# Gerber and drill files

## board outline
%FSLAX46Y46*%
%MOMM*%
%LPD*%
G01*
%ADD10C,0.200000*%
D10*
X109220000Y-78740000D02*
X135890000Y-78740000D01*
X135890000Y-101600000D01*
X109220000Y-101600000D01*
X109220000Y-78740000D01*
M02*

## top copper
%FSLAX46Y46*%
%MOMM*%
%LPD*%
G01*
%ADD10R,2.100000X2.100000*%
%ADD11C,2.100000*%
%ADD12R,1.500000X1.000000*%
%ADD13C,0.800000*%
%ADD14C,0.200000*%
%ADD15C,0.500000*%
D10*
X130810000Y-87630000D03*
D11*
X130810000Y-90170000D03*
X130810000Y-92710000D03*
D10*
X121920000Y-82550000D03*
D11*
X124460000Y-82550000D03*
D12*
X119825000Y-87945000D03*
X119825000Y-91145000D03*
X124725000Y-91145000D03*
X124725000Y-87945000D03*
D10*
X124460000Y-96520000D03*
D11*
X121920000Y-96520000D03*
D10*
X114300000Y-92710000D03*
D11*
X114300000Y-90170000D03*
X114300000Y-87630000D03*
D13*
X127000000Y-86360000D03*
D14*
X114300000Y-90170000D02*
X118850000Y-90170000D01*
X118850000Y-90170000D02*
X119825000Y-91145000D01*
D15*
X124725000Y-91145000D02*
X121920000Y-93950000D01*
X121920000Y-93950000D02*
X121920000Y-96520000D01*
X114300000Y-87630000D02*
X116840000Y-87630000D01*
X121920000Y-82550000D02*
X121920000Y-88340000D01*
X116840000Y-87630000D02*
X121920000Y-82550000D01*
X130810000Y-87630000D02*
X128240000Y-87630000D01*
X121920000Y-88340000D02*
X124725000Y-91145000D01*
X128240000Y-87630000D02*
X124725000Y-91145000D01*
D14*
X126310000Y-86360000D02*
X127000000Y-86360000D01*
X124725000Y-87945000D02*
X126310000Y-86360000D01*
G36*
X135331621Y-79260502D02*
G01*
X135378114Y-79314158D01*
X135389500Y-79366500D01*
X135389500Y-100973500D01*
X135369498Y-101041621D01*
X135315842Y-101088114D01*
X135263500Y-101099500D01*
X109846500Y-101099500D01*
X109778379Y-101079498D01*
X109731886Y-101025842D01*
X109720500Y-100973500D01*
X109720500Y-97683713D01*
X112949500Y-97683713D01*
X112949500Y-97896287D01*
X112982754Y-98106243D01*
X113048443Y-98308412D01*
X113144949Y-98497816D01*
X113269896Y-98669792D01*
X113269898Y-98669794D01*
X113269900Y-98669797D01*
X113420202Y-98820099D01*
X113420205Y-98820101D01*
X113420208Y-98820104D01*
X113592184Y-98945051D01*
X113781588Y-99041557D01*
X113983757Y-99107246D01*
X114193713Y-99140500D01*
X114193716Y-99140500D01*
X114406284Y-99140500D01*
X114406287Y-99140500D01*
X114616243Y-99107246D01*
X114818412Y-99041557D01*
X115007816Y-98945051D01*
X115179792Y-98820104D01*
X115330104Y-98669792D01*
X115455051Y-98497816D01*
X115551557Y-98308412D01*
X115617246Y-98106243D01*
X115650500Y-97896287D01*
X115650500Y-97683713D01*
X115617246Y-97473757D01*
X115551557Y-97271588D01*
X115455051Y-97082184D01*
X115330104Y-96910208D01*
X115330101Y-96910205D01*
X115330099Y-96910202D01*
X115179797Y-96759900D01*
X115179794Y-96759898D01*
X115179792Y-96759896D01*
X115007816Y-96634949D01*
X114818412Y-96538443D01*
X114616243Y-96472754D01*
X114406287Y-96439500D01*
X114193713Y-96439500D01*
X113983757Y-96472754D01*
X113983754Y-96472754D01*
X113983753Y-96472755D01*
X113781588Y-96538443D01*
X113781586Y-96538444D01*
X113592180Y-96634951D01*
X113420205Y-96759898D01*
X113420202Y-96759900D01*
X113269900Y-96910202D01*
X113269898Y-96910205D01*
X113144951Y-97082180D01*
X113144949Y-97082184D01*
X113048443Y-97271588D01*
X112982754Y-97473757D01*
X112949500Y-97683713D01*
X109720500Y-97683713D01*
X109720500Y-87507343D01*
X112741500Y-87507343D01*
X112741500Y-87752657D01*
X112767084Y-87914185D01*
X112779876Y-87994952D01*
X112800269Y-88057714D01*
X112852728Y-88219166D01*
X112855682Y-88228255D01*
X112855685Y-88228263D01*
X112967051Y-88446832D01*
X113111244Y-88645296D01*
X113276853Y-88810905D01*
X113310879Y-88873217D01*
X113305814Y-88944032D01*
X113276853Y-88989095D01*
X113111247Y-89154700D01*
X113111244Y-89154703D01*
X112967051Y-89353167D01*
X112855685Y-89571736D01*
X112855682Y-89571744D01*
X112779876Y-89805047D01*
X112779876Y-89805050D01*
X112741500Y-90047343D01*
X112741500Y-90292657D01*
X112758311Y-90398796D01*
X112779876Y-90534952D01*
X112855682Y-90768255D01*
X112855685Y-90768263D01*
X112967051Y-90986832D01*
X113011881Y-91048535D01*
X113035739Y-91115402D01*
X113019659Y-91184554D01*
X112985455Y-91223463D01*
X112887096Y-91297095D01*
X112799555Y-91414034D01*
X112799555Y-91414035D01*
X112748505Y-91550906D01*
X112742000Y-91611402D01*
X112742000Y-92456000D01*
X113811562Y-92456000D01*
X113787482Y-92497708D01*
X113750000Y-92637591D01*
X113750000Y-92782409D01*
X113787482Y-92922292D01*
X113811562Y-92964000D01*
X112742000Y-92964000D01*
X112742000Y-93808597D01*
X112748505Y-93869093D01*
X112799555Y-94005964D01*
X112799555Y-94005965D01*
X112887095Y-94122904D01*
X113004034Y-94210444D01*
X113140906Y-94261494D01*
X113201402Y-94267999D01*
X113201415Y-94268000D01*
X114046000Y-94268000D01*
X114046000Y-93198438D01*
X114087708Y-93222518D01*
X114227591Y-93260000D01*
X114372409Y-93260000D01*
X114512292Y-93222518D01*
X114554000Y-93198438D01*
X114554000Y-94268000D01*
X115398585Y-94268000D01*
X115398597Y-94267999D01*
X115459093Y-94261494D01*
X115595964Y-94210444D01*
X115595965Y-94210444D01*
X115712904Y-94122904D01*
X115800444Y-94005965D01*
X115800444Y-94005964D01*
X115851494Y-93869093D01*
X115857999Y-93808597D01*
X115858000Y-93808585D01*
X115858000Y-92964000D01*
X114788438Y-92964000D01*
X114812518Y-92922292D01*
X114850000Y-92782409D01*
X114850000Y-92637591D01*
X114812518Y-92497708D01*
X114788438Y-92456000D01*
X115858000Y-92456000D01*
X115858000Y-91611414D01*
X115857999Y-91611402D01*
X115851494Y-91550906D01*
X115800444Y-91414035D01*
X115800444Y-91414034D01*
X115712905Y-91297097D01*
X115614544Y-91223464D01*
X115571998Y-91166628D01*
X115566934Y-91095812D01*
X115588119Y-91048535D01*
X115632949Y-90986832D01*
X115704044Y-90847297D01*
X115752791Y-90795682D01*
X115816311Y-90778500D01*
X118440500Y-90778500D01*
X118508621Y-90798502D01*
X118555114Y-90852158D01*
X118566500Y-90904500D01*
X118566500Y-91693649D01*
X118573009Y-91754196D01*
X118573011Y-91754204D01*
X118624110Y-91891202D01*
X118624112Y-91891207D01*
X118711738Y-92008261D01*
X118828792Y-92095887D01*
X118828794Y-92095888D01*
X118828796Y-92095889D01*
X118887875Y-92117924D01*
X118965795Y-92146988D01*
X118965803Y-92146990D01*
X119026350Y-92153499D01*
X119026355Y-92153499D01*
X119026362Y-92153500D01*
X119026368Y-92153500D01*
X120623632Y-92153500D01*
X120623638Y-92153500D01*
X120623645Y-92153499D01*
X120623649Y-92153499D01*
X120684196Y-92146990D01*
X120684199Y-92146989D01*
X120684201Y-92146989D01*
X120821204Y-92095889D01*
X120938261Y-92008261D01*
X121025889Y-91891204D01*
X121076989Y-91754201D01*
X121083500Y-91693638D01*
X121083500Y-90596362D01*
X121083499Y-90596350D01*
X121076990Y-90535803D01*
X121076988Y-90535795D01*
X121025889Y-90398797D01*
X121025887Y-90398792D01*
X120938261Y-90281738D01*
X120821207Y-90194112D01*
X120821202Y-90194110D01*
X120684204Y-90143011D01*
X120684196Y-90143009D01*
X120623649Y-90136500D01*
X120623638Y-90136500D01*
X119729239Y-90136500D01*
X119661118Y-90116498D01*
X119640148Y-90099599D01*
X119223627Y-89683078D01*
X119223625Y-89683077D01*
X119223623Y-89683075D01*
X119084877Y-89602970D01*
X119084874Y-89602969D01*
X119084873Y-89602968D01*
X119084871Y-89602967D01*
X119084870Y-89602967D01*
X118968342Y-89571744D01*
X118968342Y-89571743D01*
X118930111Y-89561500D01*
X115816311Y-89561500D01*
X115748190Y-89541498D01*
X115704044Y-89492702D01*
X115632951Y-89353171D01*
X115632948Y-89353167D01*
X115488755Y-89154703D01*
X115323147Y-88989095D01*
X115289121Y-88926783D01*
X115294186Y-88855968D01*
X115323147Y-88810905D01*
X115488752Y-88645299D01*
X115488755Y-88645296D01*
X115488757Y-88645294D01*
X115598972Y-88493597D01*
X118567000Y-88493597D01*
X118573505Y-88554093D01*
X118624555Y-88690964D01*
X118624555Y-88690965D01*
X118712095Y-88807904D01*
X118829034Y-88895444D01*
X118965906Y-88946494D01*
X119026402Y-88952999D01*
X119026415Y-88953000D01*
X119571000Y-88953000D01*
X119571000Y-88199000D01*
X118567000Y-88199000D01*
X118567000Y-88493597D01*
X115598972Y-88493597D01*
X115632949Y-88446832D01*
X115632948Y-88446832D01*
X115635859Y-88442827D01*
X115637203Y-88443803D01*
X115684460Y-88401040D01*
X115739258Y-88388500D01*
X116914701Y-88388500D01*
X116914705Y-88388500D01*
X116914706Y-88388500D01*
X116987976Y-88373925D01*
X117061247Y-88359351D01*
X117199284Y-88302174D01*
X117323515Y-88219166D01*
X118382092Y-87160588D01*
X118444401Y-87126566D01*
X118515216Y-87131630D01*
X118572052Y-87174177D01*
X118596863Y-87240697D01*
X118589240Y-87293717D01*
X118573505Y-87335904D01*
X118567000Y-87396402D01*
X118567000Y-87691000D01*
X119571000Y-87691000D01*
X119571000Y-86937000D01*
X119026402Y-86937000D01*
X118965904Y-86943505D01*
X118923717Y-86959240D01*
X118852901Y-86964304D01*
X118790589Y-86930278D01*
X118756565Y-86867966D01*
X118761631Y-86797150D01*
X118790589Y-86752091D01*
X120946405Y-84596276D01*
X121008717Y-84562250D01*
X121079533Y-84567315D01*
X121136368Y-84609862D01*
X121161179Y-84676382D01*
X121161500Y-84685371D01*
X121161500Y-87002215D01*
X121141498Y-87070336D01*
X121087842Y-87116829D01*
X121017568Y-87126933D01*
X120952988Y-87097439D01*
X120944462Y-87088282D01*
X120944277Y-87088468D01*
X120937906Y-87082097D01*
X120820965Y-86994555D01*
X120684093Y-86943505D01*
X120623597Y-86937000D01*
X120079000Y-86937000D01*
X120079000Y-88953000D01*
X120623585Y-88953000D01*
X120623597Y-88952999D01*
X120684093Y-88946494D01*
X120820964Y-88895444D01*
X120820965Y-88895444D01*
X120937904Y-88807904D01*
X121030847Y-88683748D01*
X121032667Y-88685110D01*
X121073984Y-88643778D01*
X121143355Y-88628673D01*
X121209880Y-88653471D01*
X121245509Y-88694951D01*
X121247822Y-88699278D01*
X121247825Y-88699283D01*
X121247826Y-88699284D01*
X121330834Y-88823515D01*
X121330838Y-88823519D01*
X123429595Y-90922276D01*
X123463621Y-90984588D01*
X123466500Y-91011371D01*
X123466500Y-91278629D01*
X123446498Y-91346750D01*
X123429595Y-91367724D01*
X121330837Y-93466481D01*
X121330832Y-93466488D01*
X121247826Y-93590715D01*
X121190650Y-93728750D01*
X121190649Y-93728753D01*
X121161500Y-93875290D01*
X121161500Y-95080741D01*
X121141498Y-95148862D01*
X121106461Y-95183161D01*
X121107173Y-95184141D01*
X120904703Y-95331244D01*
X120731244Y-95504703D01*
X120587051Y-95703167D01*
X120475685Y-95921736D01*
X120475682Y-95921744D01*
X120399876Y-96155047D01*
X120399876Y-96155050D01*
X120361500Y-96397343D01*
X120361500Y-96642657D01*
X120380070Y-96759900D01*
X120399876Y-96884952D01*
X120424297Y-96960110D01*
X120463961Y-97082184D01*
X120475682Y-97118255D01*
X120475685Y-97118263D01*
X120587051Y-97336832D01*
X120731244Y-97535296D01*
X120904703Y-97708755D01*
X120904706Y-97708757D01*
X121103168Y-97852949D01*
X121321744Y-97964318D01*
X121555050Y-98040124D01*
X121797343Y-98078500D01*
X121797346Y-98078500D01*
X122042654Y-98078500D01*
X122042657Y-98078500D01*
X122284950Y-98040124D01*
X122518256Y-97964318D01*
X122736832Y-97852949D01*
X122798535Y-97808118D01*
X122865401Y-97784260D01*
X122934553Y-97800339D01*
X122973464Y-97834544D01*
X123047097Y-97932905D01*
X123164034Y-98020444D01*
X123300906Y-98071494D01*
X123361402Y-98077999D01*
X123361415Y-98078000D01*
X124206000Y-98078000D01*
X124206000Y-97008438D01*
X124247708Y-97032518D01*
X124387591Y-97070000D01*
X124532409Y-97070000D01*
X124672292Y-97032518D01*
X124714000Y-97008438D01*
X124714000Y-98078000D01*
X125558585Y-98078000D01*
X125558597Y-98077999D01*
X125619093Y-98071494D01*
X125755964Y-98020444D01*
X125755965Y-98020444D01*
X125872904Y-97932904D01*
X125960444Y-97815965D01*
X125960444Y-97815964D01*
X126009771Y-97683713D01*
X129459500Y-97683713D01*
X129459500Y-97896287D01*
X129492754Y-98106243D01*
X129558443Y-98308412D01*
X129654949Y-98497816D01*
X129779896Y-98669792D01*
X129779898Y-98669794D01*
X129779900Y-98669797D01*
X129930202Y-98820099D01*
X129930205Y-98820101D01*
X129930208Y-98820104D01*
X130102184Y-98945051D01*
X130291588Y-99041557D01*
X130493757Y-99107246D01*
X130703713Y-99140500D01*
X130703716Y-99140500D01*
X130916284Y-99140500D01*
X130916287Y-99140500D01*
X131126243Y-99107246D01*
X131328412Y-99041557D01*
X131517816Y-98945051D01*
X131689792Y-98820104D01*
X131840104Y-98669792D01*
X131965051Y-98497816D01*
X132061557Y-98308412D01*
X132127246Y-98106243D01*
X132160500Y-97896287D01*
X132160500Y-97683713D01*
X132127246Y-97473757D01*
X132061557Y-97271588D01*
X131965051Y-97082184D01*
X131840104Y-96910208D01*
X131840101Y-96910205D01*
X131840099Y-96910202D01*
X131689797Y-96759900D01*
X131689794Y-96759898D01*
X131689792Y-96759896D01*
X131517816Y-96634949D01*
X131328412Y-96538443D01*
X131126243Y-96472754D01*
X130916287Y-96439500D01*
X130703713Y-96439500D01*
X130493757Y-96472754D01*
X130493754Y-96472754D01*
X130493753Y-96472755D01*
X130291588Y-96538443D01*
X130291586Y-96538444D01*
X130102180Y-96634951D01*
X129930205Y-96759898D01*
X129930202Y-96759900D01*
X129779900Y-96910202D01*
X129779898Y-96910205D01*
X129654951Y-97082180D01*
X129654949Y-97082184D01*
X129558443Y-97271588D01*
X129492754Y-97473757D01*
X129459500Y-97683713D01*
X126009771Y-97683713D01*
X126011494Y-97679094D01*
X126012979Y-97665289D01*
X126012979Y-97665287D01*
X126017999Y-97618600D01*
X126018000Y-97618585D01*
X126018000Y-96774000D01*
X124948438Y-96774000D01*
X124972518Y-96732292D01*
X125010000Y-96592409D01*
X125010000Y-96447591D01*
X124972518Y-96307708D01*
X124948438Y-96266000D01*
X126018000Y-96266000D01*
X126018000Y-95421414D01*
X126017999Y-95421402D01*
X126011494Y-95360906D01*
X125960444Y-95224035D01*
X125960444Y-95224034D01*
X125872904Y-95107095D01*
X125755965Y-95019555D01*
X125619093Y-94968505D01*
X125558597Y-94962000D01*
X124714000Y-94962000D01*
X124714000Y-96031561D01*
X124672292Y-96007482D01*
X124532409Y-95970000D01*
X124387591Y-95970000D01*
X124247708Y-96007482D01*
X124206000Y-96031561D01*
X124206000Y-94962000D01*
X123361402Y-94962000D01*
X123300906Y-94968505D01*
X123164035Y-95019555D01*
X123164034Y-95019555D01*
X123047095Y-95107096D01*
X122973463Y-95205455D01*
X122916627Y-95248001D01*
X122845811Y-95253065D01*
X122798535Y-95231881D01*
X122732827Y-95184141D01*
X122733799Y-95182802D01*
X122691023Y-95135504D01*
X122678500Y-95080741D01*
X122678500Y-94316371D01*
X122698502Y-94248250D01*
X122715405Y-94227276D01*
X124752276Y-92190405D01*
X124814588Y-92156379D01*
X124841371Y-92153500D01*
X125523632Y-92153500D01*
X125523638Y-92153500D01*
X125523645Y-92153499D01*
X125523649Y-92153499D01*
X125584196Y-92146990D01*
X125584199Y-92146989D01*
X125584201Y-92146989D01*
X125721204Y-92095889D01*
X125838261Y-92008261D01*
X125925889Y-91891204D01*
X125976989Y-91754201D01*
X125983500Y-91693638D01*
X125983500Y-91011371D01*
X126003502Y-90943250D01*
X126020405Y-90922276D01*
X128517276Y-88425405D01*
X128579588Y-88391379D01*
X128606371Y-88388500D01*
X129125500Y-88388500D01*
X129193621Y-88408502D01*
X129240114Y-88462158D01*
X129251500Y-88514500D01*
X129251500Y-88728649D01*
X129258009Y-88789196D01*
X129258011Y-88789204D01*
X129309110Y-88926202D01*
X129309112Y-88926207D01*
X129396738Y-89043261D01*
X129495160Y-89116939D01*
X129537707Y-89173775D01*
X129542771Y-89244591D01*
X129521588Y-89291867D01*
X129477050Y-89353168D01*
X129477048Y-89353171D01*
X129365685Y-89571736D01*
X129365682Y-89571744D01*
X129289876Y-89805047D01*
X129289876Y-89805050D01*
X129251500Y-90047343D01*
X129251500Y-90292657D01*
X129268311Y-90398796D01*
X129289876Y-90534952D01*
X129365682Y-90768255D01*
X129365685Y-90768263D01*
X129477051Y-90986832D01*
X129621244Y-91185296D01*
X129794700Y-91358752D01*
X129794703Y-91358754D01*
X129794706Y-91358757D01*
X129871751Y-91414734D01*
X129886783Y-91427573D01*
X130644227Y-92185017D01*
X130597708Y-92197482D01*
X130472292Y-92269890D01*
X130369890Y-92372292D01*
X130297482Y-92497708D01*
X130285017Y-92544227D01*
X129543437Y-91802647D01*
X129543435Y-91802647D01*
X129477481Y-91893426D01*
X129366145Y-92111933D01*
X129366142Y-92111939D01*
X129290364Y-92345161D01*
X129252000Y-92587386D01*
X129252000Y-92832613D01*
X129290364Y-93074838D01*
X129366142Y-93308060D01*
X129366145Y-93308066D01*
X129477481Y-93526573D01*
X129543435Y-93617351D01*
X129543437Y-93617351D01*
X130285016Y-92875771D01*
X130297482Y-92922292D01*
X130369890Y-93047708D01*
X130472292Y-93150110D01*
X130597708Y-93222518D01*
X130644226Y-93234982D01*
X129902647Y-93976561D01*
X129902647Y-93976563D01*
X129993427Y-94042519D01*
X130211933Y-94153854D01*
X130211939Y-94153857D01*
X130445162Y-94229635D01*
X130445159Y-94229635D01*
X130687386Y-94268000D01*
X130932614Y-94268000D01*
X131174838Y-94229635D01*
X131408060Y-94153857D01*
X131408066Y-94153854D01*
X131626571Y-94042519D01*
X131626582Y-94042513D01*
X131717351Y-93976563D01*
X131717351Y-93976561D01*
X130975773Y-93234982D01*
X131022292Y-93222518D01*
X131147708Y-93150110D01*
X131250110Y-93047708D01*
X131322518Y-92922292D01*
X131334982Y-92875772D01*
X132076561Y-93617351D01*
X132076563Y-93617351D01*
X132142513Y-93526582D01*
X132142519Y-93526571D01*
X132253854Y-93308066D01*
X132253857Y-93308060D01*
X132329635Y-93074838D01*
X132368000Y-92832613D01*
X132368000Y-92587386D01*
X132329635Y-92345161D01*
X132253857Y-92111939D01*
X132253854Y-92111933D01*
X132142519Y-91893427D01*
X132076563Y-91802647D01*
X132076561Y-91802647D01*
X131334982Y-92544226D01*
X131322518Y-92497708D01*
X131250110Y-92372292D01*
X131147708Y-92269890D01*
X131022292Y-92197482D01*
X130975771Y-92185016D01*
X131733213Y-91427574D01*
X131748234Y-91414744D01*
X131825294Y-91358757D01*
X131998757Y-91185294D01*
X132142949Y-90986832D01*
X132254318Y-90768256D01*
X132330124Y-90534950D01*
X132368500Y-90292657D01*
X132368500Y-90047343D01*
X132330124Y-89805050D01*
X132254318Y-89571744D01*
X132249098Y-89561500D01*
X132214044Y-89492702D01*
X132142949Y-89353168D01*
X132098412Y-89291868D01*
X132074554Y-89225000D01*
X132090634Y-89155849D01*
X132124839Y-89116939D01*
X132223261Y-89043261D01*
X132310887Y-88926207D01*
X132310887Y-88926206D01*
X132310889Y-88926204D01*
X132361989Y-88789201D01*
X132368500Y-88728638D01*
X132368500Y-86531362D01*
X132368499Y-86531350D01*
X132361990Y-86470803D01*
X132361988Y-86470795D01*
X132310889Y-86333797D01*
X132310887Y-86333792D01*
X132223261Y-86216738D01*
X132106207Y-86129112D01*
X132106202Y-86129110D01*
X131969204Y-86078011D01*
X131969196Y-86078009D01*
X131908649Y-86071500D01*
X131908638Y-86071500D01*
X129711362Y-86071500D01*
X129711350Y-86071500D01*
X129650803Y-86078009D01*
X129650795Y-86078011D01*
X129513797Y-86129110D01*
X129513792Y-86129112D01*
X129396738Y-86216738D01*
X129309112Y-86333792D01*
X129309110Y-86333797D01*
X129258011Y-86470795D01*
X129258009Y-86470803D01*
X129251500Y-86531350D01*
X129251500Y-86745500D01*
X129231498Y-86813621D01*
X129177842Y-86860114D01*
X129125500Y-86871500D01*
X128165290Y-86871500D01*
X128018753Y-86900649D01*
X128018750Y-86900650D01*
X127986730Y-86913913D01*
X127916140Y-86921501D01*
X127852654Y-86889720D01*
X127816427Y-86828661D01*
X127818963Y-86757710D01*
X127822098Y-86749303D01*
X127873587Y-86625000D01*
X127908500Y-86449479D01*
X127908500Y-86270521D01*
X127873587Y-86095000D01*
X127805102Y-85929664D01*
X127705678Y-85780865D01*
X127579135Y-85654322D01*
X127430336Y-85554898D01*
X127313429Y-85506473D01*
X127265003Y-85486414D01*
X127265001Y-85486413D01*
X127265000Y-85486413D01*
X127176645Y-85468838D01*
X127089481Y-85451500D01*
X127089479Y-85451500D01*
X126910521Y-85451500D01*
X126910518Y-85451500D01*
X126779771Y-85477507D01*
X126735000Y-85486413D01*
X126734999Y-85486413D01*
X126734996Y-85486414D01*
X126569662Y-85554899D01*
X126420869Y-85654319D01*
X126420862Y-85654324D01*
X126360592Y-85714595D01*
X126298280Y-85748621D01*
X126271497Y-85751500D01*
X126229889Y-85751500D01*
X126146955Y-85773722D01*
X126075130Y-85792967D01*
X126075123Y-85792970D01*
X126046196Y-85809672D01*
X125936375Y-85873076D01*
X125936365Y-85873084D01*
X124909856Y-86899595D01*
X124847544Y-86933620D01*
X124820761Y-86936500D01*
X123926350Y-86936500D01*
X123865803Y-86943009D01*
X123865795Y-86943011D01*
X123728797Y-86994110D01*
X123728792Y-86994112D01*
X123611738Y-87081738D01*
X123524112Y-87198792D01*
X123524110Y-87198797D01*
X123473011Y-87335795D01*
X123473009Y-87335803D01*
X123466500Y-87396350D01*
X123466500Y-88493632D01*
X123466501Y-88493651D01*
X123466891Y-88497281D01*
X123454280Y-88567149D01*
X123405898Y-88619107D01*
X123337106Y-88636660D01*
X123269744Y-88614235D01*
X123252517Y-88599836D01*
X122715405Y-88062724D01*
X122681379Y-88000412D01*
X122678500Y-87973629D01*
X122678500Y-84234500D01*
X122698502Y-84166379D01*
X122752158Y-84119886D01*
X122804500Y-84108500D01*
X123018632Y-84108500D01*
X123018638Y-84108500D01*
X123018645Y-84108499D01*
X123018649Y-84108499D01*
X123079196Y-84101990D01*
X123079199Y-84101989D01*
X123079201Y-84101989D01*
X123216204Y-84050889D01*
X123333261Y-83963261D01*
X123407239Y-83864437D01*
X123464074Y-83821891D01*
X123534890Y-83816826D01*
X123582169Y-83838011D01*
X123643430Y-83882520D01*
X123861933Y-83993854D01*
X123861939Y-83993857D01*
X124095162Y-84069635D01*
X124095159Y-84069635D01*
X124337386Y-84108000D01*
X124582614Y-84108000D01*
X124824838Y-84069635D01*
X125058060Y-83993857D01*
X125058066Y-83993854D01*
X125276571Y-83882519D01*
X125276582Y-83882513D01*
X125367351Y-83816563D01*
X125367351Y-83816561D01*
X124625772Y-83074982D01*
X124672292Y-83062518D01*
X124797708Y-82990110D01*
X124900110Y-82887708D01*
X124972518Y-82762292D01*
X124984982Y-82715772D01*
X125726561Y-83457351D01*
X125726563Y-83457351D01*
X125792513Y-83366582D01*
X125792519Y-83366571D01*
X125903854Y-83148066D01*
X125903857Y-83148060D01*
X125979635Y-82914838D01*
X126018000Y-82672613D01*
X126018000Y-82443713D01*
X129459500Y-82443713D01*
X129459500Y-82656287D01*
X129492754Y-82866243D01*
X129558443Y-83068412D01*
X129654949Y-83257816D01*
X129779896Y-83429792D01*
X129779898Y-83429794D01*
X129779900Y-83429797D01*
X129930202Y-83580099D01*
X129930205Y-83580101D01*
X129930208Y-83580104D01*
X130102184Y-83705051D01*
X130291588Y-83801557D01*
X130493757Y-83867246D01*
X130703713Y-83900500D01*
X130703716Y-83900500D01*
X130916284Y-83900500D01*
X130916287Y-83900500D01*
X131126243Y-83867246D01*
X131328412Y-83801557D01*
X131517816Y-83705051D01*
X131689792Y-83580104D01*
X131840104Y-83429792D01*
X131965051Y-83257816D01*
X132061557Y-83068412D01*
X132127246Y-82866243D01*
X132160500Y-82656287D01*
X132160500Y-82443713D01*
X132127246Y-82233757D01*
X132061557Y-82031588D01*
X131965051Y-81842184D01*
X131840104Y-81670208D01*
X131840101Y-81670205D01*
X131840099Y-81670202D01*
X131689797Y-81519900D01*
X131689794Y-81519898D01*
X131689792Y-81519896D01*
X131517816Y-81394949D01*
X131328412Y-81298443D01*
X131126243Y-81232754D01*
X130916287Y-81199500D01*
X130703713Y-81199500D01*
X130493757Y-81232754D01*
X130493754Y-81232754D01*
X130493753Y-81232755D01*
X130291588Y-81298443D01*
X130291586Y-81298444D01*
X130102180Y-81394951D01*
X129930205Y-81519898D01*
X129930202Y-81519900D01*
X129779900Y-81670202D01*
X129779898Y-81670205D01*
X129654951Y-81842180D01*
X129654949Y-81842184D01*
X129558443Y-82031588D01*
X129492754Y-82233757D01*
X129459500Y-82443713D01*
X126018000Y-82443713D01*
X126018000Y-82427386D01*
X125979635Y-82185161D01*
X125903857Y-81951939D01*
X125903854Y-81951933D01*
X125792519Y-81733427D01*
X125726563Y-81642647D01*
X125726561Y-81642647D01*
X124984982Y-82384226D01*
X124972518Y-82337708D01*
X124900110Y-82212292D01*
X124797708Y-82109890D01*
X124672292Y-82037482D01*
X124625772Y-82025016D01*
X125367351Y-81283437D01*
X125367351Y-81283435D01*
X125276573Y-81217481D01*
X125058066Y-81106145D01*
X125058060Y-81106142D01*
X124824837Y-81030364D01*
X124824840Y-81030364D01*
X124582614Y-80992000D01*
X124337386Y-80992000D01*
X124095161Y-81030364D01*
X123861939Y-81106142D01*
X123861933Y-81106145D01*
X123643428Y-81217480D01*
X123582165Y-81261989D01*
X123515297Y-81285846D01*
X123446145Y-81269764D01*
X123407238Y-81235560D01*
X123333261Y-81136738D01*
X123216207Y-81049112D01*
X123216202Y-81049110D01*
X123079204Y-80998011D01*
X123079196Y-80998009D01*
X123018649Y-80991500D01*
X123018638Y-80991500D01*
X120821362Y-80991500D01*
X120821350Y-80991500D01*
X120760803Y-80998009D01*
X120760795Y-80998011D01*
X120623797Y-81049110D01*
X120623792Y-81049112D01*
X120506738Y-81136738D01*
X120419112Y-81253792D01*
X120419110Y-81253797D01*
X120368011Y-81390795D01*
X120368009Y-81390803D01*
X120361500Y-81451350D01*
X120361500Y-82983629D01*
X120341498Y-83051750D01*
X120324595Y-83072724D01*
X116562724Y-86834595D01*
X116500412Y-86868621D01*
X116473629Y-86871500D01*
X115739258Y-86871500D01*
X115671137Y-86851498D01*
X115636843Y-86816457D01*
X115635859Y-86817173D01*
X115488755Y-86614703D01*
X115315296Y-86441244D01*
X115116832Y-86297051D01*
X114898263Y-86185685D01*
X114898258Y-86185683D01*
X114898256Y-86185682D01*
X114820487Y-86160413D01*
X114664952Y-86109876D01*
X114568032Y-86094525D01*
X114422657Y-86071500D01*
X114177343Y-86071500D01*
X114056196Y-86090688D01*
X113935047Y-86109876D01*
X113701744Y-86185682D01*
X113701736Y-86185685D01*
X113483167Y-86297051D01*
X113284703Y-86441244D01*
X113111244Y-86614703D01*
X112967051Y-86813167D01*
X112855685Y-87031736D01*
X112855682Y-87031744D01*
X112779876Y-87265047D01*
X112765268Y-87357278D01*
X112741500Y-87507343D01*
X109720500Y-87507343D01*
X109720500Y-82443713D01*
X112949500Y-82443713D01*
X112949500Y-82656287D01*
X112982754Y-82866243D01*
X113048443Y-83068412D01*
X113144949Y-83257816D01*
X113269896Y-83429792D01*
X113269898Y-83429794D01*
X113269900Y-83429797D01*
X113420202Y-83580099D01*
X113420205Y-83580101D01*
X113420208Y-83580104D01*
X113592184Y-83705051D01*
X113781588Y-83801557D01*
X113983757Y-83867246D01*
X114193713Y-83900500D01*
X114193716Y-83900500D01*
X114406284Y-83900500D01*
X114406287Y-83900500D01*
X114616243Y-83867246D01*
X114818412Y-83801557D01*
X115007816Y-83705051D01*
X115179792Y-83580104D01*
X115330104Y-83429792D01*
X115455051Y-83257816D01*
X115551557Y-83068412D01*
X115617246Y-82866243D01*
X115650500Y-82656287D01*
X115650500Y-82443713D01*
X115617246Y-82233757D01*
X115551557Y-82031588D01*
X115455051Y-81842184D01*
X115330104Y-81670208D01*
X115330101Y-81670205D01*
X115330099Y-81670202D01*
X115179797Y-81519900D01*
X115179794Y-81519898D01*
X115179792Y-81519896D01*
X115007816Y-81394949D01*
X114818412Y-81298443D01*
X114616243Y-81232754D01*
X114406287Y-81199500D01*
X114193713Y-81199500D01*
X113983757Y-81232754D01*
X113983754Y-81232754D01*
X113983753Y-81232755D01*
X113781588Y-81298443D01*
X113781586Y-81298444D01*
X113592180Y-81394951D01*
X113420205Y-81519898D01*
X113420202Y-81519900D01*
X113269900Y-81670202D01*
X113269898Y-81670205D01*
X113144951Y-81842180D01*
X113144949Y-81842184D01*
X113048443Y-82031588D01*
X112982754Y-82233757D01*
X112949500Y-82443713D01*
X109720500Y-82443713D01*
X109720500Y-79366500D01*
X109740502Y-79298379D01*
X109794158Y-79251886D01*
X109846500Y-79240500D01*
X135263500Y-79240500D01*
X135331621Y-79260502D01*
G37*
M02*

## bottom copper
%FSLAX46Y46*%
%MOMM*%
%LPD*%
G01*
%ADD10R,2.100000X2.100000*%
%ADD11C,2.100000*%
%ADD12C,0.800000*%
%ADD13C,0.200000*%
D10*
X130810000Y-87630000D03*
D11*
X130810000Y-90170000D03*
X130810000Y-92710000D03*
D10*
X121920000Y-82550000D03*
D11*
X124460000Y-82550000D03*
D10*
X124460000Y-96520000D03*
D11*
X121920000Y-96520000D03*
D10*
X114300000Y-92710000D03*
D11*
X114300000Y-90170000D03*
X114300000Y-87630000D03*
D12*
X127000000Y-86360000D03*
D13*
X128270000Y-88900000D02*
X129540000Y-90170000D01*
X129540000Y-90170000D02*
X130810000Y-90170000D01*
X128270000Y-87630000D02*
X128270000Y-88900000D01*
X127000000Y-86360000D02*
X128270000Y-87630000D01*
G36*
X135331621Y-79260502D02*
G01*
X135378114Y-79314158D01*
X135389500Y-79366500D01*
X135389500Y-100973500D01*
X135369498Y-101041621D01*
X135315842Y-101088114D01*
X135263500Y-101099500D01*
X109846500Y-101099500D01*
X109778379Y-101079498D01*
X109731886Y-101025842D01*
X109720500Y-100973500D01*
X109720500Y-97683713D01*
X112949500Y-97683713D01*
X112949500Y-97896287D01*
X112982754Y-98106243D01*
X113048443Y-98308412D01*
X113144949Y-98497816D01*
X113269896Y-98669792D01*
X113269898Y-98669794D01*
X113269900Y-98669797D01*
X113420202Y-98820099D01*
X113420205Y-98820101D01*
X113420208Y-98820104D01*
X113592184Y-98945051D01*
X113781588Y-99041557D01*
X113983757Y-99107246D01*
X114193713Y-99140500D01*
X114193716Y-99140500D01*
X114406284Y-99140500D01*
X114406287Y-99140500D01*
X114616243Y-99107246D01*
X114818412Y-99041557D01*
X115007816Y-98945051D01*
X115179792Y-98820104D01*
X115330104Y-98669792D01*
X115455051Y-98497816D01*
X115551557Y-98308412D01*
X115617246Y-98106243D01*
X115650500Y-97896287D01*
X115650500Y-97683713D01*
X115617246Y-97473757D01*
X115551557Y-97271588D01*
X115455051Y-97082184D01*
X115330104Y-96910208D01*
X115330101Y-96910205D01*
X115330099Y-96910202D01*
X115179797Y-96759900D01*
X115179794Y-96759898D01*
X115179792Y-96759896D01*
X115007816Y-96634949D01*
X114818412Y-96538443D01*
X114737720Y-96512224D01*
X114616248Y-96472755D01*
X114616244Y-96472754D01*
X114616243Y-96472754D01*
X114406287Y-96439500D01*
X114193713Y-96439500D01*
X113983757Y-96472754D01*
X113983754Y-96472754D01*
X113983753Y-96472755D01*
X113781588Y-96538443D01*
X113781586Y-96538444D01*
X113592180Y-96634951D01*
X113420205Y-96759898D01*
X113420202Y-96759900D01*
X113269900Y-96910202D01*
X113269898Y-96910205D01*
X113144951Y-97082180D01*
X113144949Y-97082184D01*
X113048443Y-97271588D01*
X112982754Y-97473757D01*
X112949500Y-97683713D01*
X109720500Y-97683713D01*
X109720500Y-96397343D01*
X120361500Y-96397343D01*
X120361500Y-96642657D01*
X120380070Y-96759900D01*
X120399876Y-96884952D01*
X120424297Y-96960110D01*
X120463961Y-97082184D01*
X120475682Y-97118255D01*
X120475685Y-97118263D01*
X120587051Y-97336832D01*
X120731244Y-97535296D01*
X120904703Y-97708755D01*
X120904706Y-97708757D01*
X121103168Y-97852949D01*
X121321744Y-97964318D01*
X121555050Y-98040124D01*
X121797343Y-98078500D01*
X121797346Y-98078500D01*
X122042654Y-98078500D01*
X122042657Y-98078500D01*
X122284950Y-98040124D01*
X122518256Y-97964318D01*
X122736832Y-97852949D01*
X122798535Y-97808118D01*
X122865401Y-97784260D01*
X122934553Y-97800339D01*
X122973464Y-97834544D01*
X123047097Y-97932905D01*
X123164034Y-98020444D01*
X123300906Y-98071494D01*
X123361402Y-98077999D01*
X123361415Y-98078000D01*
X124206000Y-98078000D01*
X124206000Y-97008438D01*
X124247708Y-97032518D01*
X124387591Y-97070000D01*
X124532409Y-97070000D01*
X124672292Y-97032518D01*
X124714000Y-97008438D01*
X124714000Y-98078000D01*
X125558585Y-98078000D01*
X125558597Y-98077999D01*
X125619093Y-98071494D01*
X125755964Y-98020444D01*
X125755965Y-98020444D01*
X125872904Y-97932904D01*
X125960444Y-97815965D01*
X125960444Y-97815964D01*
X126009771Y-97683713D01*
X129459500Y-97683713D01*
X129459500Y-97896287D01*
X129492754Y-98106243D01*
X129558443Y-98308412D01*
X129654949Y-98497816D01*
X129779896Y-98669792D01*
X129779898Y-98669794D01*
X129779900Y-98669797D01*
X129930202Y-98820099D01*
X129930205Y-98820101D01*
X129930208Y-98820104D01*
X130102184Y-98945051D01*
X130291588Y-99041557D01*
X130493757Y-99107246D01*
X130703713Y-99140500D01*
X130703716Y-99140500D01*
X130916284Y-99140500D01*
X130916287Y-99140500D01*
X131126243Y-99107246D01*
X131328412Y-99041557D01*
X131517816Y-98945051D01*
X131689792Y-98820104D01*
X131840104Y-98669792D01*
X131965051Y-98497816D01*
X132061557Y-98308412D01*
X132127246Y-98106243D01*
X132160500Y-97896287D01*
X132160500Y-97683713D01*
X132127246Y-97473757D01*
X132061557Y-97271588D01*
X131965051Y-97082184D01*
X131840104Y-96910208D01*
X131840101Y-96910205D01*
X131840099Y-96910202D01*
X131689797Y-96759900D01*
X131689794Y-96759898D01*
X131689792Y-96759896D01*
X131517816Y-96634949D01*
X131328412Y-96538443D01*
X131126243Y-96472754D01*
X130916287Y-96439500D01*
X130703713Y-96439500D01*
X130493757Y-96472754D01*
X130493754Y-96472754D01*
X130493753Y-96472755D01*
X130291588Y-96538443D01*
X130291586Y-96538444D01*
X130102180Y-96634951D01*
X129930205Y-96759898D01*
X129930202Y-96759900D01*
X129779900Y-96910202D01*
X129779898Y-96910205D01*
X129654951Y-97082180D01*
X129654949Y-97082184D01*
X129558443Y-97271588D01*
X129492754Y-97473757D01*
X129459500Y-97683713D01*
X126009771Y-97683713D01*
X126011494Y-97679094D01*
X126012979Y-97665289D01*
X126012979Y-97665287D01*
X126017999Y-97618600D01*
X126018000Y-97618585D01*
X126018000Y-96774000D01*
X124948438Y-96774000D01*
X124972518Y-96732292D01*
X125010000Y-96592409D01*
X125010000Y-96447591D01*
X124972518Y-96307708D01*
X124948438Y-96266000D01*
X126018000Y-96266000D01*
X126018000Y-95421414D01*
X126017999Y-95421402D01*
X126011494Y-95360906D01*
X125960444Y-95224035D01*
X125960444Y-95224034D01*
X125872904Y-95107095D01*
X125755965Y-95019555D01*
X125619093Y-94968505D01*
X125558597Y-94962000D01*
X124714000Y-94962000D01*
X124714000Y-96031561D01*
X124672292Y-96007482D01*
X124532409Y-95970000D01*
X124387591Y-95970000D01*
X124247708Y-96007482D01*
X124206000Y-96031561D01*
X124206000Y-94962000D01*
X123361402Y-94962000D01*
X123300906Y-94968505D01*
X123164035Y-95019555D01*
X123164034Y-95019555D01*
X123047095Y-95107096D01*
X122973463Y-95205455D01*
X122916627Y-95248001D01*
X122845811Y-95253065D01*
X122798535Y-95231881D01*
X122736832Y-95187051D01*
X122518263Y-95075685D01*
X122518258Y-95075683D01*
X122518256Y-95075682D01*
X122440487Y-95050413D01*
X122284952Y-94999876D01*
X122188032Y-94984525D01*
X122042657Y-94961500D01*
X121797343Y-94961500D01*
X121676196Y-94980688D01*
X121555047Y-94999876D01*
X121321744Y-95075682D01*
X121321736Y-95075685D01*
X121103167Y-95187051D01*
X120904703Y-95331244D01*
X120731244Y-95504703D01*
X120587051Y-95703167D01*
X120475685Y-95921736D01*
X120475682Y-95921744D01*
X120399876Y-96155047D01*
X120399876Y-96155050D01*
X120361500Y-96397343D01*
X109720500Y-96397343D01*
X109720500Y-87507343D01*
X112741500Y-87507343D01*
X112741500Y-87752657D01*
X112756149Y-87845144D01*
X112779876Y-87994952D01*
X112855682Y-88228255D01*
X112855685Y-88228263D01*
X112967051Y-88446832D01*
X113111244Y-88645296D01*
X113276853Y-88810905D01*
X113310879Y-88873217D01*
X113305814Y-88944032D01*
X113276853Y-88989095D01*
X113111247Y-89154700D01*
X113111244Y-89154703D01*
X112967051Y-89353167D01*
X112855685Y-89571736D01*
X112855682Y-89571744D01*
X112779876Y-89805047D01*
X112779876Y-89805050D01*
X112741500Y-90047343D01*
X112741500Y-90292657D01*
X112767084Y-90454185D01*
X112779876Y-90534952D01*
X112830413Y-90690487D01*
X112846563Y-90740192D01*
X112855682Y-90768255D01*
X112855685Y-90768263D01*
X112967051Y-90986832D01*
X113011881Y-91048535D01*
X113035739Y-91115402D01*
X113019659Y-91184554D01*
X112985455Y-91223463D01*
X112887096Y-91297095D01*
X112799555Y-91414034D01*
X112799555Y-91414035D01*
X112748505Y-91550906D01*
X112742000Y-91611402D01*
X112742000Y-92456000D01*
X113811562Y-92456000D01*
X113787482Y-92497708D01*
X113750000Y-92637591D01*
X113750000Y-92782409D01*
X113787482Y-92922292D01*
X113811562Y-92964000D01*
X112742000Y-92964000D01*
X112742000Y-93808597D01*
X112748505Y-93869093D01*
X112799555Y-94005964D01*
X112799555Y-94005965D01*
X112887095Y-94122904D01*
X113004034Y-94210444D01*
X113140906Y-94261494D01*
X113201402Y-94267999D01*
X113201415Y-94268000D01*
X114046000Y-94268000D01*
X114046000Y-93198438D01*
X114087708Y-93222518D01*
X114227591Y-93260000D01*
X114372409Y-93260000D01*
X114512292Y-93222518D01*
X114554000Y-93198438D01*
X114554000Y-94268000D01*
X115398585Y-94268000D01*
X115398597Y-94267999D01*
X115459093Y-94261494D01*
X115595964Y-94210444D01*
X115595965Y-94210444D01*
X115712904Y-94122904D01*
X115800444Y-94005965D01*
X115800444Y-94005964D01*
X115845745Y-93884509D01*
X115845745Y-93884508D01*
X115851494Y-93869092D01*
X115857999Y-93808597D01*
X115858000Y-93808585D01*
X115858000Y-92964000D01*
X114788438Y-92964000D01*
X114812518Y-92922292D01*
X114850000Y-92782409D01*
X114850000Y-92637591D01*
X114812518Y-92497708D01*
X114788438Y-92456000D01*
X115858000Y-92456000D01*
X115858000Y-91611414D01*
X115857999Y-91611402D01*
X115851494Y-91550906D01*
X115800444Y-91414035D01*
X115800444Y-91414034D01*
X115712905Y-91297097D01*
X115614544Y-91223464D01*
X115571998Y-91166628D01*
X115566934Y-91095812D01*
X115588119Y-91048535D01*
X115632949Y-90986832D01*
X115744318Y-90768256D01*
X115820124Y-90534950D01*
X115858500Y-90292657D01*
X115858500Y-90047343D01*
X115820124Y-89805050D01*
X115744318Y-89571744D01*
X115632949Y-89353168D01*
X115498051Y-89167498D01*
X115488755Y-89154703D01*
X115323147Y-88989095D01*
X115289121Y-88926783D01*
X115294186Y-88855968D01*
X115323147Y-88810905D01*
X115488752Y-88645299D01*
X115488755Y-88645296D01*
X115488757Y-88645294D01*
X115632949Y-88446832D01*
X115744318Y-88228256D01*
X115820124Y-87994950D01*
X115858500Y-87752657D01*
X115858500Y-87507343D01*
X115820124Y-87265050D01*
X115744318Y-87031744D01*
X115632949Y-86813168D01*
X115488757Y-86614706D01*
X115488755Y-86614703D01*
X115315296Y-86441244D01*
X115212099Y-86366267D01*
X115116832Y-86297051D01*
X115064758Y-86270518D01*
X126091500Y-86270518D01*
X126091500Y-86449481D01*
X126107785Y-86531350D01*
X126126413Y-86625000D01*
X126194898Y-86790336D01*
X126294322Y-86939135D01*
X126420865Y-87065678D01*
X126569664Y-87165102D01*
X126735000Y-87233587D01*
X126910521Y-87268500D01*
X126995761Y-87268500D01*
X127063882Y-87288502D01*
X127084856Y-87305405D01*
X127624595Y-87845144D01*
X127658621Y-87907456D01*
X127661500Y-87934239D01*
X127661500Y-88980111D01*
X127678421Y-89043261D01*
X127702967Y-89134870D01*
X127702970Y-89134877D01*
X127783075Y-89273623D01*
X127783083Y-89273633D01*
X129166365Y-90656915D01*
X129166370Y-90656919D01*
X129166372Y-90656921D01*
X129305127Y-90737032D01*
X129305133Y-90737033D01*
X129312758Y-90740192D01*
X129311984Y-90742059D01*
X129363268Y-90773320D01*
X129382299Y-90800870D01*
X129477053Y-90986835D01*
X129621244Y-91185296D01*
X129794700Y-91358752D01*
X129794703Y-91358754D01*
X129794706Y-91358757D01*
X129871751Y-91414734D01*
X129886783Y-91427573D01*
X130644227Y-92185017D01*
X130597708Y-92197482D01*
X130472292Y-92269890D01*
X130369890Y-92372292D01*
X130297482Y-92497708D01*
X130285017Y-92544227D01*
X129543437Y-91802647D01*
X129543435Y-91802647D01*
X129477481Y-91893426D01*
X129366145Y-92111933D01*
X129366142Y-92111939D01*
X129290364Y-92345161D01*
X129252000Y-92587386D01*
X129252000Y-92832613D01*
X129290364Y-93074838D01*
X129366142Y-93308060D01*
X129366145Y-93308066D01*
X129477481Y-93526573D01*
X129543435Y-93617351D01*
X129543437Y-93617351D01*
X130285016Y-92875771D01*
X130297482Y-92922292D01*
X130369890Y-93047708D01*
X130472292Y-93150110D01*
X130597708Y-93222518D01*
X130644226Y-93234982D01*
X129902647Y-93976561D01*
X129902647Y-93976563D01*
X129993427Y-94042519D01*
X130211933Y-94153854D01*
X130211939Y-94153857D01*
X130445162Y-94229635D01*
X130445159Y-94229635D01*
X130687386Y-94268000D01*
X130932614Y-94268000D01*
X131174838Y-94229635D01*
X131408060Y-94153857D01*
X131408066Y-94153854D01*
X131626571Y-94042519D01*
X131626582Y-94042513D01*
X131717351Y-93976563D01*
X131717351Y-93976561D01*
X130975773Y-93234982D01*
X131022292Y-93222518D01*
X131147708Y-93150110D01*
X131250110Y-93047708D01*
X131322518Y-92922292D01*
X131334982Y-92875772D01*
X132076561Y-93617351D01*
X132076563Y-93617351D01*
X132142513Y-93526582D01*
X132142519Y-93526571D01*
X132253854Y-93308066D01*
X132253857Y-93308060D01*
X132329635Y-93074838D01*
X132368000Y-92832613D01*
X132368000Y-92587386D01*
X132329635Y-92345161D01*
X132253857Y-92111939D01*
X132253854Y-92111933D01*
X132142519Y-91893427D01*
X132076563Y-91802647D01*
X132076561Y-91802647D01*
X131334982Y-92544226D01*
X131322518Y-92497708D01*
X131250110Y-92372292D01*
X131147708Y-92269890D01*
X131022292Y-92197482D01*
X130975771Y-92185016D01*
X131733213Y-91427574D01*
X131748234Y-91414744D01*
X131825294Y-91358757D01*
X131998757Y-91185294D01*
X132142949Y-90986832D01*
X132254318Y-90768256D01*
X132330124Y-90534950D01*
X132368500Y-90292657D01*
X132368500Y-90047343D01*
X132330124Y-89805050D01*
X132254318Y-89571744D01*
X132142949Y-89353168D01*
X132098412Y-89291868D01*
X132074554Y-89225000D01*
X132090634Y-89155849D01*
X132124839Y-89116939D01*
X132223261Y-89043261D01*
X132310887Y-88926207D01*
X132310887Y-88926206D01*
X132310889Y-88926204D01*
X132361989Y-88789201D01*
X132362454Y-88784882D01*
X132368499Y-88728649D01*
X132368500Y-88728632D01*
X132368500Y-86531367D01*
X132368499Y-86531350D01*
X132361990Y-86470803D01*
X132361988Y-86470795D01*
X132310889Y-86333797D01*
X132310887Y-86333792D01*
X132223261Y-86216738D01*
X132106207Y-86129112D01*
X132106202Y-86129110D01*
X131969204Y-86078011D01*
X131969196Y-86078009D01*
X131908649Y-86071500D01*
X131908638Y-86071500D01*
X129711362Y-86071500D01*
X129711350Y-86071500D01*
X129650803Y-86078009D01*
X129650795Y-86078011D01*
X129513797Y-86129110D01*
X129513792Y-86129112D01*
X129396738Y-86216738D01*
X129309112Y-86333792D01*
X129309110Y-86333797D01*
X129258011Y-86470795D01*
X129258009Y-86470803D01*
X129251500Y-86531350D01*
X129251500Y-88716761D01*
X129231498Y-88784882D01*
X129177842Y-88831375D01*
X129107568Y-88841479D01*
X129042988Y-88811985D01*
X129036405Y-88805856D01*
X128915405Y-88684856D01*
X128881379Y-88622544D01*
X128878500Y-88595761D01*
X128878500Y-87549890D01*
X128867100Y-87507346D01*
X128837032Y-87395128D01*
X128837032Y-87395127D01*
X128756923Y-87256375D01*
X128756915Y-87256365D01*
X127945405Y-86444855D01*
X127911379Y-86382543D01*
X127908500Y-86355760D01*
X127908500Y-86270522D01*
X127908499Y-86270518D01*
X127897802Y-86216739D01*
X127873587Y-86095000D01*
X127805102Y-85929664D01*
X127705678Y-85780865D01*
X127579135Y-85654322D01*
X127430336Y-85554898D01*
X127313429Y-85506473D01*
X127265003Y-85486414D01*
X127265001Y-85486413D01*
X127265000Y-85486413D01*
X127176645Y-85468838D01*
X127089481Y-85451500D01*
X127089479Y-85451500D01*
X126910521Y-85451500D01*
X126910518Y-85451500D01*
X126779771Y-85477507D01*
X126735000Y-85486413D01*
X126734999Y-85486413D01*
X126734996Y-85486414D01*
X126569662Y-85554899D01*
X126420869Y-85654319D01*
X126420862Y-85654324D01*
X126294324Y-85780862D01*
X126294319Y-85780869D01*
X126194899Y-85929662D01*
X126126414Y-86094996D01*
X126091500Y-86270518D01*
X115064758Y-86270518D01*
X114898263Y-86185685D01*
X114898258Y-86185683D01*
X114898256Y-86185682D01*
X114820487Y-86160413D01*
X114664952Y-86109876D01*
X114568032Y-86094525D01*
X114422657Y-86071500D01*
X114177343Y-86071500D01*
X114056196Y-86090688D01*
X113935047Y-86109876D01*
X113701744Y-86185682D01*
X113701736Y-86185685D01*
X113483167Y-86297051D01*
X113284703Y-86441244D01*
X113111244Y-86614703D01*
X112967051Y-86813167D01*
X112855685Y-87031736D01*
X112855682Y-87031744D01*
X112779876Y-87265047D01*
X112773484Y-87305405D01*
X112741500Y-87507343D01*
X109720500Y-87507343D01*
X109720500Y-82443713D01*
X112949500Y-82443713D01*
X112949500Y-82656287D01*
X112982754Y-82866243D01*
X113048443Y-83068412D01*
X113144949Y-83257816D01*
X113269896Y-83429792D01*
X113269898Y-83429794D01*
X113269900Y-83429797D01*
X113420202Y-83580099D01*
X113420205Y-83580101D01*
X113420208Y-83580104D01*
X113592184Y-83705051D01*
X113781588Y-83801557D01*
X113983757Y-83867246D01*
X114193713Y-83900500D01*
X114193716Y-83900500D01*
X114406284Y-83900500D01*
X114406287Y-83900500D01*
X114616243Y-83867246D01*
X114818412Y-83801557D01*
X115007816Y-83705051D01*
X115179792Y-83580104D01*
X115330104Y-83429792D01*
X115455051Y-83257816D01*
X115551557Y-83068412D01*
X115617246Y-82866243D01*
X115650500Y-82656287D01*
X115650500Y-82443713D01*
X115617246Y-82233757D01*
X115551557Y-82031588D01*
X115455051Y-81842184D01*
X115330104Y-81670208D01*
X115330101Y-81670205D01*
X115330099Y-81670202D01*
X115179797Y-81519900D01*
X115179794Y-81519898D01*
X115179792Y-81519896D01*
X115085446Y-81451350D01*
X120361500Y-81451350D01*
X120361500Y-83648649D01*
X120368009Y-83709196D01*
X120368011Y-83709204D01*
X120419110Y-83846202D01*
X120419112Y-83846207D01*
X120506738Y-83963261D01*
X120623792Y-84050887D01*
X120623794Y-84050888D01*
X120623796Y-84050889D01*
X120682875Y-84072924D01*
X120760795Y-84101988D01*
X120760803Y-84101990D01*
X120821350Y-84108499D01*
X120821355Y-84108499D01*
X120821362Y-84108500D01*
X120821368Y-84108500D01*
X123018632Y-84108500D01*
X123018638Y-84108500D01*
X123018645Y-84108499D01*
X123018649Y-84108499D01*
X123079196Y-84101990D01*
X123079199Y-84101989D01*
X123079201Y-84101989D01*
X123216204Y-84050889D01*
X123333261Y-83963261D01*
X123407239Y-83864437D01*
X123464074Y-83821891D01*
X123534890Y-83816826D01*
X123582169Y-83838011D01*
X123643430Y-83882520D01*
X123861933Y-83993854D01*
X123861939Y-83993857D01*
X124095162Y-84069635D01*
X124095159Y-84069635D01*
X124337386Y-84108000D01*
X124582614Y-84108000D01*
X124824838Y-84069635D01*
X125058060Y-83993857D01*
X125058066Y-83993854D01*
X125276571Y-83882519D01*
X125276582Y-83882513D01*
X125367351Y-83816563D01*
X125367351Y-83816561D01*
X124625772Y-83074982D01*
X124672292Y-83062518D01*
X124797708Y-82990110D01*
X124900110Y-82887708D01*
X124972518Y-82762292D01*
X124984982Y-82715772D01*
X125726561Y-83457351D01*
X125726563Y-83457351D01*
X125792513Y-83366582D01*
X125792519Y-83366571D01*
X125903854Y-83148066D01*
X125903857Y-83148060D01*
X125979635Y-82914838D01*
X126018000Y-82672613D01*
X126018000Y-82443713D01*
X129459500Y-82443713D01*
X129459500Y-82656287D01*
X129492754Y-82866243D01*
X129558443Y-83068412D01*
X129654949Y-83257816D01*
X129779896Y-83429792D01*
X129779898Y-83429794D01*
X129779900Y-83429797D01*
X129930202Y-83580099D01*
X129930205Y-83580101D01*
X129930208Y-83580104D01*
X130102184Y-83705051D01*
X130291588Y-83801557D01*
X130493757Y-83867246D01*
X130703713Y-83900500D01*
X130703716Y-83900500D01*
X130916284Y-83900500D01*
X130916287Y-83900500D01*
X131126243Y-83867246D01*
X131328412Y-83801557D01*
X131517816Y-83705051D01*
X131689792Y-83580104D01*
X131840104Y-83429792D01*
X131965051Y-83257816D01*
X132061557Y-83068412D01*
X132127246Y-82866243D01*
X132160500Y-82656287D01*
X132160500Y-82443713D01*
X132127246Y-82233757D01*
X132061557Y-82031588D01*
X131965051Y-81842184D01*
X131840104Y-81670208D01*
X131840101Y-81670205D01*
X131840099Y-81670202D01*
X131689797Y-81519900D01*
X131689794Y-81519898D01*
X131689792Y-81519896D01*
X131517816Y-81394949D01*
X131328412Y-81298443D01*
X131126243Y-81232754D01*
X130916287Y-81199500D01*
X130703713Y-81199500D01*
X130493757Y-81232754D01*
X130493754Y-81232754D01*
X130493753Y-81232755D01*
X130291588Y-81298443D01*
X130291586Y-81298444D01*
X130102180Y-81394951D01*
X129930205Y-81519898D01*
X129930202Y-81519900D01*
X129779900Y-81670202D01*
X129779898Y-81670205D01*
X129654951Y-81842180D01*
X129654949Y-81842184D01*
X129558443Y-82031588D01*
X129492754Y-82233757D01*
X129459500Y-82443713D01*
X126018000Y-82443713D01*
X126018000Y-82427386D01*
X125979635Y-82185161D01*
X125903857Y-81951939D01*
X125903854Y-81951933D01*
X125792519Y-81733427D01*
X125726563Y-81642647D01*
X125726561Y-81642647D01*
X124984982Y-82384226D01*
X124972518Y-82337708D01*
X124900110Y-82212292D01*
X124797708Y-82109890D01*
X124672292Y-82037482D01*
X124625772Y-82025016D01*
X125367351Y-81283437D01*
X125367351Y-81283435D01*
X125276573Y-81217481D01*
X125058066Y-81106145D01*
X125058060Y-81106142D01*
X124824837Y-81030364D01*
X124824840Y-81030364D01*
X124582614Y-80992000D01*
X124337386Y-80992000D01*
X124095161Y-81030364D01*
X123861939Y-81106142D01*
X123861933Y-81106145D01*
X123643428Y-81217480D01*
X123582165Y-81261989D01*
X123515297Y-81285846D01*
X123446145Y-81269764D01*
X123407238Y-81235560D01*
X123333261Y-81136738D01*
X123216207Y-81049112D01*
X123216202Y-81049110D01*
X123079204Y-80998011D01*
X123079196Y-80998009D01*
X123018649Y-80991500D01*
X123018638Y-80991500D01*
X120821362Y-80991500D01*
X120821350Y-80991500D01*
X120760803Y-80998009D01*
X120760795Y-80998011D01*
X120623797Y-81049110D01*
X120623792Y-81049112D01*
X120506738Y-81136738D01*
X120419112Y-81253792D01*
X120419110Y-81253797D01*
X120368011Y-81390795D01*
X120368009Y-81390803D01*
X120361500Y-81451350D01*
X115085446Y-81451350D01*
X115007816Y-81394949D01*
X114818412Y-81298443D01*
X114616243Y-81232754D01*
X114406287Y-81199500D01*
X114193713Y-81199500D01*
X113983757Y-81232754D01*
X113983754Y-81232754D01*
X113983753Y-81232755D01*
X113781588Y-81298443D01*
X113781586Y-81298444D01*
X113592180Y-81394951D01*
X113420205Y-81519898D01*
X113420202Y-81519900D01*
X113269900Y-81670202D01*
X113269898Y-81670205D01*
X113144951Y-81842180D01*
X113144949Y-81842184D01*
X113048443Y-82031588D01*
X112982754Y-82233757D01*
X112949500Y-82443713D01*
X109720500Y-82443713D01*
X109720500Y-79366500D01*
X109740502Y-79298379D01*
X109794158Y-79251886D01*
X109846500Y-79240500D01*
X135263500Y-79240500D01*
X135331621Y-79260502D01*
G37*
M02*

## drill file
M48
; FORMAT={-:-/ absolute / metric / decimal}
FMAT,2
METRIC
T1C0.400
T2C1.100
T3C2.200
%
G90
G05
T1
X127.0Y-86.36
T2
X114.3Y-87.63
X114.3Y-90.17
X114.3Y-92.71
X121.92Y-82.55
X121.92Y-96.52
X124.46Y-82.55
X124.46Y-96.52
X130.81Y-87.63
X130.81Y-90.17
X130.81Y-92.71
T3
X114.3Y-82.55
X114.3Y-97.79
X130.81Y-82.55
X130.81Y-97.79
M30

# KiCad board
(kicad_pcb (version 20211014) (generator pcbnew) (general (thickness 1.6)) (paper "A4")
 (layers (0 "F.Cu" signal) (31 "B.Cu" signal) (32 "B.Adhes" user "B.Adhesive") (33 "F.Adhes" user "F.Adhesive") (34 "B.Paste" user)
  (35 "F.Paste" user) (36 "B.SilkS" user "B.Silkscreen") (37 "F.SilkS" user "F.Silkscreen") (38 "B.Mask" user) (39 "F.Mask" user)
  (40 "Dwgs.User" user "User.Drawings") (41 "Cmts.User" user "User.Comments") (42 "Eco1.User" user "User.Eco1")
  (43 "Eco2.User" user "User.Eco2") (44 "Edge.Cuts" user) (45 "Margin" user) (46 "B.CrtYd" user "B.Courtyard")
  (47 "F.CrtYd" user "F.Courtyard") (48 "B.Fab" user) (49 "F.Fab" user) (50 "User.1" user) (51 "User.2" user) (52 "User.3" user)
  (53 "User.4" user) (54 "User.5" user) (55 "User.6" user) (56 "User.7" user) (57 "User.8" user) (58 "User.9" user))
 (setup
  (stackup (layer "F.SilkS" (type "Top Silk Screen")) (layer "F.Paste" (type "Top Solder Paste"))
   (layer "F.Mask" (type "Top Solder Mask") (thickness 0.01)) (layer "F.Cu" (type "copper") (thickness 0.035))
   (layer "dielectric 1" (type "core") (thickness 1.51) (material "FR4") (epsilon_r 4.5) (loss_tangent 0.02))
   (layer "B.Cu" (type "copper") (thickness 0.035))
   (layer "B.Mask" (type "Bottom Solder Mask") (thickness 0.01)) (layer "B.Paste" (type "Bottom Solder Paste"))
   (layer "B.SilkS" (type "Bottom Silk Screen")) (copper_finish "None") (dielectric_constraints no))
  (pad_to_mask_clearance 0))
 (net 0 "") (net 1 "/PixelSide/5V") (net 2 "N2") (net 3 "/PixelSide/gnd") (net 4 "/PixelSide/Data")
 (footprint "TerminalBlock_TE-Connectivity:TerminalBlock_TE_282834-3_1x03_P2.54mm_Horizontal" (layer "F.Cu") (at 130.81 87.63 -90)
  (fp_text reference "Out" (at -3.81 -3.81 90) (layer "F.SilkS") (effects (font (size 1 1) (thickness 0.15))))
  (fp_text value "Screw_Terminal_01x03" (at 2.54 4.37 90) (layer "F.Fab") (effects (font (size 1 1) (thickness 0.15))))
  (pad "1" thru_hole rect (at 0 0 270) (size 2.1 2.1) (drill 1.1) (layers *.Cu *.Mask) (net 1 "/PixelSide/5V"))
  (pad "2" thru_hole circle (at 2.54 0 270) (size 2.1 2.1) (drill 1.1) (layers *.Cu *.Mask) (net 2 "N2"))
  (pad "3" thru_hole circle (at 5.08 0 270) (size 2.1 2.1) (drill 1.1) (layers *.Cu *.Mask) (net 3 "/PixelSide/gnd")))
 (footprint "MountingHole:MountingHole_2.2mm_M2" (layer "F.Cu") (at 130.81 97.79)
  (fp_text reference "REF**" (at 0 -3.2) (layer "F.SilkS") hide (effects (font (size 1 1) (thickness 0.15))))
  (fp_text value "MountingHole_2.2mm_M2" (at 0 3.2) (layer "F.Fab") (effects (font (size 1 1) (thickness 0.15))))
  (pad "" np_thru_hole circle (at 0 0) (size 2.2 2.2) (drill 2.2) (layers *.Cu *.Mask)))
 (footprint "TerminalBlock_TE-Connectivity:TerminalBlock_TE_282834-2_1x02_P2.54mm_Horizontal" (layer "F.Cu") (at 121.92 82.55)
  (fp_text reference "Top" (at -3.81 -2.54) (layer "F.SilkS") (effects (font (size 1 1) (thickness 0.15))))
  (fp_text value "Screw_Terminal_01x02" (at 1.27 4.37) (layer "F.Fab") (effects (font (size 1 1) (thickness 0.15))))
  (pad "1" thru_hole rect (at 0 0) (size 2.1 2.1) (drill 1.1) (layers *.Cu *.Mask) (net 1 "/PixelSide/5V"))
  (pad "2" thru_hole circle (at 2.54 0) (size 2.1 2.1) (drill 1.1) (layers *.Cu *.Mask) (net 3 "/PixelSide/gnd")))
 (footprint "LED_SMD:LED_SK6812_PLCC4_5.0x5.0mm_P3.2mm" (layer "F.Cu") (at 122.275 89.545 180)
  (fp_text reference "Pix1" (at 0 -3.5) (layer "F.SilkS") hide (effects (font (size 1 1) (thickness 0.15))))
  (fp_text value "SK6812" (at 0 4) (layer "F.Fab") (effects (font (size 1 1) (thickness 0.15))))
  (pad "1" smd rect (at 2.45 1.6 180) (size 1.5 1) (layers "F.Cu" "F.Paste" "F.Mask") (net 3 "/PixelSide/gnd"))
  (pad "2" smd rect (at 2.45 -1.6 180) (size 1.5 1) (layers "F.Cu" "F.Paste" "F.Mask") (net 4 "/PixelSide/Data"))
  (pad "3" smd rect (at -2.45 -1.6 180) (size 1.5 1) (layers "F.Cu" "F.Paste" "F.Mask") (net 1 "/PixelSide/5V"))
  (pad "4" smd rect (at -2.45 1.6 180) (size 1.5 1) (layers "F.Cu" "F.Paste" "F.Mask") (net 2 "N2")))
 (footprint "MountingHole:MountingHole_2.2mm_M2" (layer "F.Cu") (at 114.3 82.55)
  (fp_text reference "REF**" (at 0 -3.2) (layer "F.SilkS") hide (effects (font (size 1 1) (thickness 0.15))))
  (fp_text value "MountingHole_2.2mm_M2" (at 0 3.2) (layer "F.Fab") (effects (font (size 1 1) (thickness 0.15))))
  (pad "" np_thru_hole circle (at 0 0) (size 2.2 2.2) (drill 2.2) (layers *.Cu *.Mask)))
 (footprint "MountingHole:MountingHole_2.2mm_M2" (layer "F.Cu") (at 130.81 82.55)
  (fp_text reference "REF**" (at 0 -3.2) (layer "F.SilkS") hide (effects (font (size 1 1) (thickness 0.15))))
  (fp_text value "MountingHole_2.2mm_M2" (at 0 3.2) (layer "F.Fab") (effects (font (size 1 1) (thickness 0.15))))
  (pad "" np_thru_hole circle (at 0 0) (size 2.2 2.2) (drill 2.2) (layers *.Cu *.Mask)))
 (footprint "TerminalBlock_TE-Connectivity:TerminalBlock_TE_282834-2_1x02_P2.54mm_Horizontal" (layer "F.Cu") (at 124.46 96.52 180)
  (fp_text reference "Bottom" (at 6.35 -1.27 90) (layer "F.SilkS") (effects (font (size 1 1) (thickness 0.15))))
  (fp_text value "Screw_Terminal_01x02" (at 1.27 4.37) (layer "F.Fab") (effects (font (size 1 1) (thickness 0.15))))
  (pad "1" thru_hole rect (at 0 0 180) (size 2.1 2.1) (drill 1.1) (layers *.Cu *.Mask) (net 3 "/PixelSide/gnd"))
  (pad "2" thru_hole circle (at 2.54 0 180) (size 2.1 2.1) (drill 1.1) (layers *.Cu *.Mask) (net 1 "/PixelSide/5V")))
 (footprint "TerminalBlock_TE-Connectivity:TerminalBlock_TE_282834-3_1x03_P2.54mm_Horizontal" (layer "F.Cu") (at 114.3 92.71 90)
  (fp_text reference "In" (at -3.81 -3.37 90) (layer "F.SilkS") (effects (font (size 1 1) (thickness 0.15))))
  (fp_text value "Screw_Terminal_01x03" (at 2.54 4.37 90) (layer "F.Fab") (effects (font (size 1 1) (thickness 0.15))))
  (pad "1" thru_hole rect (at 0 0 90) (size 2.1 2.1) (drill 1.1) (layers *.Cu *.Mask) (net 3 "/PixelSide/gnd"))
  (pad "2" thru_hole circle (at 2.54 0 90) (size 2.1 2.1) (drill 1.1) (layers *.Cu *.Mask) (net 4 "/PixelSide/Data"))
  (pad "3" thru_hole circle (at 5.08 0 90) (size 2.1 2.1) (drill 1.1) (layers *.Cu *.Mask) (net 1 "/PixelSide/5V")))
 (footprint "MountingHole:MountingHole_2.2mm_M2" (layer "F.Cu") (at 114.3 97.79)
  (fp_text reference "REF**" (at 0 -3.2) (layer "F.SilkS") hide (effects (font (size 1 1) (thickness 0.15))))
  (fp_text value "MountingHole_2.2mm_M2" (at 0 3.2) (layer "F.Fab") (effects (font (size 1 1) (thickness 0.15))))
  (pad "" np_thru_hole circle (at 0 0) (size 2.2 2.2) (drill 2.2) (layers *.Cu *.Mask)))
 (gr_rect (start 109.22 78.74) (end 135.89 101.6) (layer "Edge.Cuts") (width 0.2) (fill none))
 (segment (start 114.3 90.17) (end 118.85 90.17) (width 0.2) (layer "F.Cu") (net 4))
 (segment (start 118.85 90.17) (end 119.825 91.145) (width 0.2) (layer "F.Cu") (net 4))
 (segment (start 124.725 91.145) (end 121.92 93.95) (width 0.5) (layer "F.Cu") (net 1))
 (segment (start 121.92 93.95) (end 121.92 96.52) (width 0.5) (layer "F.Cu") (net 1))
 (segment (start 114.3 87.63) (end 116.84 87.63) (width 0.5) (layer "F.Cu") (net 1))
 (segment (start 121.92 82.55) (end 121.92 88.34) (width 0.5) (layer "F.Cu") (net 1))
 (segment (start 116.84 87.63) (end 121.92 82.55) (width 0.5) (layer "F.Cu") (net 1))
 (segment (start 130.81 87.63) (end 128.24 87.63) (width 0.5) (layer "F.Cu") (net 1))
 (segment (start 121.92 88.34) (end 124.725 91.145) (width 0.5) (layer "F.Cu") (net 1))
 (segment (start 128.24 87.63) (end 124.725 91.145) (width 0.5) (layer "F.Cu") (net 1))
 (segment (start 126.31 86.36) (end 127 86.36) (width 0.2) (layer "F.Cu") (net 2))
 (segment (start 124.725 87.945) (end 126.31 86.36) (width 0.2) (layer "F.Cu") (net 2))
 (via (at 127 86.36) (size 0.8) (drill 0.4) (layers "F.Cu" "B.Cu") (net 2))
 (segment (start 128.27 88.9) (end 129.54 90.17) (width 0.2) (layer "B.Cu") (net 2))
 (segment (start 129.54 90.17) (end 130.81 90.17) (width 0.2) (layer "B.Cu") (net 2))
 (segment (start 128.27 87.63) (end 128.27 88.9) (width 0.2) (layer "B.Cu") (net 2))
 (segment (start 127 86.36) (end 128.27 87.63) (width 0.2) (layer "B.Cu") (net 2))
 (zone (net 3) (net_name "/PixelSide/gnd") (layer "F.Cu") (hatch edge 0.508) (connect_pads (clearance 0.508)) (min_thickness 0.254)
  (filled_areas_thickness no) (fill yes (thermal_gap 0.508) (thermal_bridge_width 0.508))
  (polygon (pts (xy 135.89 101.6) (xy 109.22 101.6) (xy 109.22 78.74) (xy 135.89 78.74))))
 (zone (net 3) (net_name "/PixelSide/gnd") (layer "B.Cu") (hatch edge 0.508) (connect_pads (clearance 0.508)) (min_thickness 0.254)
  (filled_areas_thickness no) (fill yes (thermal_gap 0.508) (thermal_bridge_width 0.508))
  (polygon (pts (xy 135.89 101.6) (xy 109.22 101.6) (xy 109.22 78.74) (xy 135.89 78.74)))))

